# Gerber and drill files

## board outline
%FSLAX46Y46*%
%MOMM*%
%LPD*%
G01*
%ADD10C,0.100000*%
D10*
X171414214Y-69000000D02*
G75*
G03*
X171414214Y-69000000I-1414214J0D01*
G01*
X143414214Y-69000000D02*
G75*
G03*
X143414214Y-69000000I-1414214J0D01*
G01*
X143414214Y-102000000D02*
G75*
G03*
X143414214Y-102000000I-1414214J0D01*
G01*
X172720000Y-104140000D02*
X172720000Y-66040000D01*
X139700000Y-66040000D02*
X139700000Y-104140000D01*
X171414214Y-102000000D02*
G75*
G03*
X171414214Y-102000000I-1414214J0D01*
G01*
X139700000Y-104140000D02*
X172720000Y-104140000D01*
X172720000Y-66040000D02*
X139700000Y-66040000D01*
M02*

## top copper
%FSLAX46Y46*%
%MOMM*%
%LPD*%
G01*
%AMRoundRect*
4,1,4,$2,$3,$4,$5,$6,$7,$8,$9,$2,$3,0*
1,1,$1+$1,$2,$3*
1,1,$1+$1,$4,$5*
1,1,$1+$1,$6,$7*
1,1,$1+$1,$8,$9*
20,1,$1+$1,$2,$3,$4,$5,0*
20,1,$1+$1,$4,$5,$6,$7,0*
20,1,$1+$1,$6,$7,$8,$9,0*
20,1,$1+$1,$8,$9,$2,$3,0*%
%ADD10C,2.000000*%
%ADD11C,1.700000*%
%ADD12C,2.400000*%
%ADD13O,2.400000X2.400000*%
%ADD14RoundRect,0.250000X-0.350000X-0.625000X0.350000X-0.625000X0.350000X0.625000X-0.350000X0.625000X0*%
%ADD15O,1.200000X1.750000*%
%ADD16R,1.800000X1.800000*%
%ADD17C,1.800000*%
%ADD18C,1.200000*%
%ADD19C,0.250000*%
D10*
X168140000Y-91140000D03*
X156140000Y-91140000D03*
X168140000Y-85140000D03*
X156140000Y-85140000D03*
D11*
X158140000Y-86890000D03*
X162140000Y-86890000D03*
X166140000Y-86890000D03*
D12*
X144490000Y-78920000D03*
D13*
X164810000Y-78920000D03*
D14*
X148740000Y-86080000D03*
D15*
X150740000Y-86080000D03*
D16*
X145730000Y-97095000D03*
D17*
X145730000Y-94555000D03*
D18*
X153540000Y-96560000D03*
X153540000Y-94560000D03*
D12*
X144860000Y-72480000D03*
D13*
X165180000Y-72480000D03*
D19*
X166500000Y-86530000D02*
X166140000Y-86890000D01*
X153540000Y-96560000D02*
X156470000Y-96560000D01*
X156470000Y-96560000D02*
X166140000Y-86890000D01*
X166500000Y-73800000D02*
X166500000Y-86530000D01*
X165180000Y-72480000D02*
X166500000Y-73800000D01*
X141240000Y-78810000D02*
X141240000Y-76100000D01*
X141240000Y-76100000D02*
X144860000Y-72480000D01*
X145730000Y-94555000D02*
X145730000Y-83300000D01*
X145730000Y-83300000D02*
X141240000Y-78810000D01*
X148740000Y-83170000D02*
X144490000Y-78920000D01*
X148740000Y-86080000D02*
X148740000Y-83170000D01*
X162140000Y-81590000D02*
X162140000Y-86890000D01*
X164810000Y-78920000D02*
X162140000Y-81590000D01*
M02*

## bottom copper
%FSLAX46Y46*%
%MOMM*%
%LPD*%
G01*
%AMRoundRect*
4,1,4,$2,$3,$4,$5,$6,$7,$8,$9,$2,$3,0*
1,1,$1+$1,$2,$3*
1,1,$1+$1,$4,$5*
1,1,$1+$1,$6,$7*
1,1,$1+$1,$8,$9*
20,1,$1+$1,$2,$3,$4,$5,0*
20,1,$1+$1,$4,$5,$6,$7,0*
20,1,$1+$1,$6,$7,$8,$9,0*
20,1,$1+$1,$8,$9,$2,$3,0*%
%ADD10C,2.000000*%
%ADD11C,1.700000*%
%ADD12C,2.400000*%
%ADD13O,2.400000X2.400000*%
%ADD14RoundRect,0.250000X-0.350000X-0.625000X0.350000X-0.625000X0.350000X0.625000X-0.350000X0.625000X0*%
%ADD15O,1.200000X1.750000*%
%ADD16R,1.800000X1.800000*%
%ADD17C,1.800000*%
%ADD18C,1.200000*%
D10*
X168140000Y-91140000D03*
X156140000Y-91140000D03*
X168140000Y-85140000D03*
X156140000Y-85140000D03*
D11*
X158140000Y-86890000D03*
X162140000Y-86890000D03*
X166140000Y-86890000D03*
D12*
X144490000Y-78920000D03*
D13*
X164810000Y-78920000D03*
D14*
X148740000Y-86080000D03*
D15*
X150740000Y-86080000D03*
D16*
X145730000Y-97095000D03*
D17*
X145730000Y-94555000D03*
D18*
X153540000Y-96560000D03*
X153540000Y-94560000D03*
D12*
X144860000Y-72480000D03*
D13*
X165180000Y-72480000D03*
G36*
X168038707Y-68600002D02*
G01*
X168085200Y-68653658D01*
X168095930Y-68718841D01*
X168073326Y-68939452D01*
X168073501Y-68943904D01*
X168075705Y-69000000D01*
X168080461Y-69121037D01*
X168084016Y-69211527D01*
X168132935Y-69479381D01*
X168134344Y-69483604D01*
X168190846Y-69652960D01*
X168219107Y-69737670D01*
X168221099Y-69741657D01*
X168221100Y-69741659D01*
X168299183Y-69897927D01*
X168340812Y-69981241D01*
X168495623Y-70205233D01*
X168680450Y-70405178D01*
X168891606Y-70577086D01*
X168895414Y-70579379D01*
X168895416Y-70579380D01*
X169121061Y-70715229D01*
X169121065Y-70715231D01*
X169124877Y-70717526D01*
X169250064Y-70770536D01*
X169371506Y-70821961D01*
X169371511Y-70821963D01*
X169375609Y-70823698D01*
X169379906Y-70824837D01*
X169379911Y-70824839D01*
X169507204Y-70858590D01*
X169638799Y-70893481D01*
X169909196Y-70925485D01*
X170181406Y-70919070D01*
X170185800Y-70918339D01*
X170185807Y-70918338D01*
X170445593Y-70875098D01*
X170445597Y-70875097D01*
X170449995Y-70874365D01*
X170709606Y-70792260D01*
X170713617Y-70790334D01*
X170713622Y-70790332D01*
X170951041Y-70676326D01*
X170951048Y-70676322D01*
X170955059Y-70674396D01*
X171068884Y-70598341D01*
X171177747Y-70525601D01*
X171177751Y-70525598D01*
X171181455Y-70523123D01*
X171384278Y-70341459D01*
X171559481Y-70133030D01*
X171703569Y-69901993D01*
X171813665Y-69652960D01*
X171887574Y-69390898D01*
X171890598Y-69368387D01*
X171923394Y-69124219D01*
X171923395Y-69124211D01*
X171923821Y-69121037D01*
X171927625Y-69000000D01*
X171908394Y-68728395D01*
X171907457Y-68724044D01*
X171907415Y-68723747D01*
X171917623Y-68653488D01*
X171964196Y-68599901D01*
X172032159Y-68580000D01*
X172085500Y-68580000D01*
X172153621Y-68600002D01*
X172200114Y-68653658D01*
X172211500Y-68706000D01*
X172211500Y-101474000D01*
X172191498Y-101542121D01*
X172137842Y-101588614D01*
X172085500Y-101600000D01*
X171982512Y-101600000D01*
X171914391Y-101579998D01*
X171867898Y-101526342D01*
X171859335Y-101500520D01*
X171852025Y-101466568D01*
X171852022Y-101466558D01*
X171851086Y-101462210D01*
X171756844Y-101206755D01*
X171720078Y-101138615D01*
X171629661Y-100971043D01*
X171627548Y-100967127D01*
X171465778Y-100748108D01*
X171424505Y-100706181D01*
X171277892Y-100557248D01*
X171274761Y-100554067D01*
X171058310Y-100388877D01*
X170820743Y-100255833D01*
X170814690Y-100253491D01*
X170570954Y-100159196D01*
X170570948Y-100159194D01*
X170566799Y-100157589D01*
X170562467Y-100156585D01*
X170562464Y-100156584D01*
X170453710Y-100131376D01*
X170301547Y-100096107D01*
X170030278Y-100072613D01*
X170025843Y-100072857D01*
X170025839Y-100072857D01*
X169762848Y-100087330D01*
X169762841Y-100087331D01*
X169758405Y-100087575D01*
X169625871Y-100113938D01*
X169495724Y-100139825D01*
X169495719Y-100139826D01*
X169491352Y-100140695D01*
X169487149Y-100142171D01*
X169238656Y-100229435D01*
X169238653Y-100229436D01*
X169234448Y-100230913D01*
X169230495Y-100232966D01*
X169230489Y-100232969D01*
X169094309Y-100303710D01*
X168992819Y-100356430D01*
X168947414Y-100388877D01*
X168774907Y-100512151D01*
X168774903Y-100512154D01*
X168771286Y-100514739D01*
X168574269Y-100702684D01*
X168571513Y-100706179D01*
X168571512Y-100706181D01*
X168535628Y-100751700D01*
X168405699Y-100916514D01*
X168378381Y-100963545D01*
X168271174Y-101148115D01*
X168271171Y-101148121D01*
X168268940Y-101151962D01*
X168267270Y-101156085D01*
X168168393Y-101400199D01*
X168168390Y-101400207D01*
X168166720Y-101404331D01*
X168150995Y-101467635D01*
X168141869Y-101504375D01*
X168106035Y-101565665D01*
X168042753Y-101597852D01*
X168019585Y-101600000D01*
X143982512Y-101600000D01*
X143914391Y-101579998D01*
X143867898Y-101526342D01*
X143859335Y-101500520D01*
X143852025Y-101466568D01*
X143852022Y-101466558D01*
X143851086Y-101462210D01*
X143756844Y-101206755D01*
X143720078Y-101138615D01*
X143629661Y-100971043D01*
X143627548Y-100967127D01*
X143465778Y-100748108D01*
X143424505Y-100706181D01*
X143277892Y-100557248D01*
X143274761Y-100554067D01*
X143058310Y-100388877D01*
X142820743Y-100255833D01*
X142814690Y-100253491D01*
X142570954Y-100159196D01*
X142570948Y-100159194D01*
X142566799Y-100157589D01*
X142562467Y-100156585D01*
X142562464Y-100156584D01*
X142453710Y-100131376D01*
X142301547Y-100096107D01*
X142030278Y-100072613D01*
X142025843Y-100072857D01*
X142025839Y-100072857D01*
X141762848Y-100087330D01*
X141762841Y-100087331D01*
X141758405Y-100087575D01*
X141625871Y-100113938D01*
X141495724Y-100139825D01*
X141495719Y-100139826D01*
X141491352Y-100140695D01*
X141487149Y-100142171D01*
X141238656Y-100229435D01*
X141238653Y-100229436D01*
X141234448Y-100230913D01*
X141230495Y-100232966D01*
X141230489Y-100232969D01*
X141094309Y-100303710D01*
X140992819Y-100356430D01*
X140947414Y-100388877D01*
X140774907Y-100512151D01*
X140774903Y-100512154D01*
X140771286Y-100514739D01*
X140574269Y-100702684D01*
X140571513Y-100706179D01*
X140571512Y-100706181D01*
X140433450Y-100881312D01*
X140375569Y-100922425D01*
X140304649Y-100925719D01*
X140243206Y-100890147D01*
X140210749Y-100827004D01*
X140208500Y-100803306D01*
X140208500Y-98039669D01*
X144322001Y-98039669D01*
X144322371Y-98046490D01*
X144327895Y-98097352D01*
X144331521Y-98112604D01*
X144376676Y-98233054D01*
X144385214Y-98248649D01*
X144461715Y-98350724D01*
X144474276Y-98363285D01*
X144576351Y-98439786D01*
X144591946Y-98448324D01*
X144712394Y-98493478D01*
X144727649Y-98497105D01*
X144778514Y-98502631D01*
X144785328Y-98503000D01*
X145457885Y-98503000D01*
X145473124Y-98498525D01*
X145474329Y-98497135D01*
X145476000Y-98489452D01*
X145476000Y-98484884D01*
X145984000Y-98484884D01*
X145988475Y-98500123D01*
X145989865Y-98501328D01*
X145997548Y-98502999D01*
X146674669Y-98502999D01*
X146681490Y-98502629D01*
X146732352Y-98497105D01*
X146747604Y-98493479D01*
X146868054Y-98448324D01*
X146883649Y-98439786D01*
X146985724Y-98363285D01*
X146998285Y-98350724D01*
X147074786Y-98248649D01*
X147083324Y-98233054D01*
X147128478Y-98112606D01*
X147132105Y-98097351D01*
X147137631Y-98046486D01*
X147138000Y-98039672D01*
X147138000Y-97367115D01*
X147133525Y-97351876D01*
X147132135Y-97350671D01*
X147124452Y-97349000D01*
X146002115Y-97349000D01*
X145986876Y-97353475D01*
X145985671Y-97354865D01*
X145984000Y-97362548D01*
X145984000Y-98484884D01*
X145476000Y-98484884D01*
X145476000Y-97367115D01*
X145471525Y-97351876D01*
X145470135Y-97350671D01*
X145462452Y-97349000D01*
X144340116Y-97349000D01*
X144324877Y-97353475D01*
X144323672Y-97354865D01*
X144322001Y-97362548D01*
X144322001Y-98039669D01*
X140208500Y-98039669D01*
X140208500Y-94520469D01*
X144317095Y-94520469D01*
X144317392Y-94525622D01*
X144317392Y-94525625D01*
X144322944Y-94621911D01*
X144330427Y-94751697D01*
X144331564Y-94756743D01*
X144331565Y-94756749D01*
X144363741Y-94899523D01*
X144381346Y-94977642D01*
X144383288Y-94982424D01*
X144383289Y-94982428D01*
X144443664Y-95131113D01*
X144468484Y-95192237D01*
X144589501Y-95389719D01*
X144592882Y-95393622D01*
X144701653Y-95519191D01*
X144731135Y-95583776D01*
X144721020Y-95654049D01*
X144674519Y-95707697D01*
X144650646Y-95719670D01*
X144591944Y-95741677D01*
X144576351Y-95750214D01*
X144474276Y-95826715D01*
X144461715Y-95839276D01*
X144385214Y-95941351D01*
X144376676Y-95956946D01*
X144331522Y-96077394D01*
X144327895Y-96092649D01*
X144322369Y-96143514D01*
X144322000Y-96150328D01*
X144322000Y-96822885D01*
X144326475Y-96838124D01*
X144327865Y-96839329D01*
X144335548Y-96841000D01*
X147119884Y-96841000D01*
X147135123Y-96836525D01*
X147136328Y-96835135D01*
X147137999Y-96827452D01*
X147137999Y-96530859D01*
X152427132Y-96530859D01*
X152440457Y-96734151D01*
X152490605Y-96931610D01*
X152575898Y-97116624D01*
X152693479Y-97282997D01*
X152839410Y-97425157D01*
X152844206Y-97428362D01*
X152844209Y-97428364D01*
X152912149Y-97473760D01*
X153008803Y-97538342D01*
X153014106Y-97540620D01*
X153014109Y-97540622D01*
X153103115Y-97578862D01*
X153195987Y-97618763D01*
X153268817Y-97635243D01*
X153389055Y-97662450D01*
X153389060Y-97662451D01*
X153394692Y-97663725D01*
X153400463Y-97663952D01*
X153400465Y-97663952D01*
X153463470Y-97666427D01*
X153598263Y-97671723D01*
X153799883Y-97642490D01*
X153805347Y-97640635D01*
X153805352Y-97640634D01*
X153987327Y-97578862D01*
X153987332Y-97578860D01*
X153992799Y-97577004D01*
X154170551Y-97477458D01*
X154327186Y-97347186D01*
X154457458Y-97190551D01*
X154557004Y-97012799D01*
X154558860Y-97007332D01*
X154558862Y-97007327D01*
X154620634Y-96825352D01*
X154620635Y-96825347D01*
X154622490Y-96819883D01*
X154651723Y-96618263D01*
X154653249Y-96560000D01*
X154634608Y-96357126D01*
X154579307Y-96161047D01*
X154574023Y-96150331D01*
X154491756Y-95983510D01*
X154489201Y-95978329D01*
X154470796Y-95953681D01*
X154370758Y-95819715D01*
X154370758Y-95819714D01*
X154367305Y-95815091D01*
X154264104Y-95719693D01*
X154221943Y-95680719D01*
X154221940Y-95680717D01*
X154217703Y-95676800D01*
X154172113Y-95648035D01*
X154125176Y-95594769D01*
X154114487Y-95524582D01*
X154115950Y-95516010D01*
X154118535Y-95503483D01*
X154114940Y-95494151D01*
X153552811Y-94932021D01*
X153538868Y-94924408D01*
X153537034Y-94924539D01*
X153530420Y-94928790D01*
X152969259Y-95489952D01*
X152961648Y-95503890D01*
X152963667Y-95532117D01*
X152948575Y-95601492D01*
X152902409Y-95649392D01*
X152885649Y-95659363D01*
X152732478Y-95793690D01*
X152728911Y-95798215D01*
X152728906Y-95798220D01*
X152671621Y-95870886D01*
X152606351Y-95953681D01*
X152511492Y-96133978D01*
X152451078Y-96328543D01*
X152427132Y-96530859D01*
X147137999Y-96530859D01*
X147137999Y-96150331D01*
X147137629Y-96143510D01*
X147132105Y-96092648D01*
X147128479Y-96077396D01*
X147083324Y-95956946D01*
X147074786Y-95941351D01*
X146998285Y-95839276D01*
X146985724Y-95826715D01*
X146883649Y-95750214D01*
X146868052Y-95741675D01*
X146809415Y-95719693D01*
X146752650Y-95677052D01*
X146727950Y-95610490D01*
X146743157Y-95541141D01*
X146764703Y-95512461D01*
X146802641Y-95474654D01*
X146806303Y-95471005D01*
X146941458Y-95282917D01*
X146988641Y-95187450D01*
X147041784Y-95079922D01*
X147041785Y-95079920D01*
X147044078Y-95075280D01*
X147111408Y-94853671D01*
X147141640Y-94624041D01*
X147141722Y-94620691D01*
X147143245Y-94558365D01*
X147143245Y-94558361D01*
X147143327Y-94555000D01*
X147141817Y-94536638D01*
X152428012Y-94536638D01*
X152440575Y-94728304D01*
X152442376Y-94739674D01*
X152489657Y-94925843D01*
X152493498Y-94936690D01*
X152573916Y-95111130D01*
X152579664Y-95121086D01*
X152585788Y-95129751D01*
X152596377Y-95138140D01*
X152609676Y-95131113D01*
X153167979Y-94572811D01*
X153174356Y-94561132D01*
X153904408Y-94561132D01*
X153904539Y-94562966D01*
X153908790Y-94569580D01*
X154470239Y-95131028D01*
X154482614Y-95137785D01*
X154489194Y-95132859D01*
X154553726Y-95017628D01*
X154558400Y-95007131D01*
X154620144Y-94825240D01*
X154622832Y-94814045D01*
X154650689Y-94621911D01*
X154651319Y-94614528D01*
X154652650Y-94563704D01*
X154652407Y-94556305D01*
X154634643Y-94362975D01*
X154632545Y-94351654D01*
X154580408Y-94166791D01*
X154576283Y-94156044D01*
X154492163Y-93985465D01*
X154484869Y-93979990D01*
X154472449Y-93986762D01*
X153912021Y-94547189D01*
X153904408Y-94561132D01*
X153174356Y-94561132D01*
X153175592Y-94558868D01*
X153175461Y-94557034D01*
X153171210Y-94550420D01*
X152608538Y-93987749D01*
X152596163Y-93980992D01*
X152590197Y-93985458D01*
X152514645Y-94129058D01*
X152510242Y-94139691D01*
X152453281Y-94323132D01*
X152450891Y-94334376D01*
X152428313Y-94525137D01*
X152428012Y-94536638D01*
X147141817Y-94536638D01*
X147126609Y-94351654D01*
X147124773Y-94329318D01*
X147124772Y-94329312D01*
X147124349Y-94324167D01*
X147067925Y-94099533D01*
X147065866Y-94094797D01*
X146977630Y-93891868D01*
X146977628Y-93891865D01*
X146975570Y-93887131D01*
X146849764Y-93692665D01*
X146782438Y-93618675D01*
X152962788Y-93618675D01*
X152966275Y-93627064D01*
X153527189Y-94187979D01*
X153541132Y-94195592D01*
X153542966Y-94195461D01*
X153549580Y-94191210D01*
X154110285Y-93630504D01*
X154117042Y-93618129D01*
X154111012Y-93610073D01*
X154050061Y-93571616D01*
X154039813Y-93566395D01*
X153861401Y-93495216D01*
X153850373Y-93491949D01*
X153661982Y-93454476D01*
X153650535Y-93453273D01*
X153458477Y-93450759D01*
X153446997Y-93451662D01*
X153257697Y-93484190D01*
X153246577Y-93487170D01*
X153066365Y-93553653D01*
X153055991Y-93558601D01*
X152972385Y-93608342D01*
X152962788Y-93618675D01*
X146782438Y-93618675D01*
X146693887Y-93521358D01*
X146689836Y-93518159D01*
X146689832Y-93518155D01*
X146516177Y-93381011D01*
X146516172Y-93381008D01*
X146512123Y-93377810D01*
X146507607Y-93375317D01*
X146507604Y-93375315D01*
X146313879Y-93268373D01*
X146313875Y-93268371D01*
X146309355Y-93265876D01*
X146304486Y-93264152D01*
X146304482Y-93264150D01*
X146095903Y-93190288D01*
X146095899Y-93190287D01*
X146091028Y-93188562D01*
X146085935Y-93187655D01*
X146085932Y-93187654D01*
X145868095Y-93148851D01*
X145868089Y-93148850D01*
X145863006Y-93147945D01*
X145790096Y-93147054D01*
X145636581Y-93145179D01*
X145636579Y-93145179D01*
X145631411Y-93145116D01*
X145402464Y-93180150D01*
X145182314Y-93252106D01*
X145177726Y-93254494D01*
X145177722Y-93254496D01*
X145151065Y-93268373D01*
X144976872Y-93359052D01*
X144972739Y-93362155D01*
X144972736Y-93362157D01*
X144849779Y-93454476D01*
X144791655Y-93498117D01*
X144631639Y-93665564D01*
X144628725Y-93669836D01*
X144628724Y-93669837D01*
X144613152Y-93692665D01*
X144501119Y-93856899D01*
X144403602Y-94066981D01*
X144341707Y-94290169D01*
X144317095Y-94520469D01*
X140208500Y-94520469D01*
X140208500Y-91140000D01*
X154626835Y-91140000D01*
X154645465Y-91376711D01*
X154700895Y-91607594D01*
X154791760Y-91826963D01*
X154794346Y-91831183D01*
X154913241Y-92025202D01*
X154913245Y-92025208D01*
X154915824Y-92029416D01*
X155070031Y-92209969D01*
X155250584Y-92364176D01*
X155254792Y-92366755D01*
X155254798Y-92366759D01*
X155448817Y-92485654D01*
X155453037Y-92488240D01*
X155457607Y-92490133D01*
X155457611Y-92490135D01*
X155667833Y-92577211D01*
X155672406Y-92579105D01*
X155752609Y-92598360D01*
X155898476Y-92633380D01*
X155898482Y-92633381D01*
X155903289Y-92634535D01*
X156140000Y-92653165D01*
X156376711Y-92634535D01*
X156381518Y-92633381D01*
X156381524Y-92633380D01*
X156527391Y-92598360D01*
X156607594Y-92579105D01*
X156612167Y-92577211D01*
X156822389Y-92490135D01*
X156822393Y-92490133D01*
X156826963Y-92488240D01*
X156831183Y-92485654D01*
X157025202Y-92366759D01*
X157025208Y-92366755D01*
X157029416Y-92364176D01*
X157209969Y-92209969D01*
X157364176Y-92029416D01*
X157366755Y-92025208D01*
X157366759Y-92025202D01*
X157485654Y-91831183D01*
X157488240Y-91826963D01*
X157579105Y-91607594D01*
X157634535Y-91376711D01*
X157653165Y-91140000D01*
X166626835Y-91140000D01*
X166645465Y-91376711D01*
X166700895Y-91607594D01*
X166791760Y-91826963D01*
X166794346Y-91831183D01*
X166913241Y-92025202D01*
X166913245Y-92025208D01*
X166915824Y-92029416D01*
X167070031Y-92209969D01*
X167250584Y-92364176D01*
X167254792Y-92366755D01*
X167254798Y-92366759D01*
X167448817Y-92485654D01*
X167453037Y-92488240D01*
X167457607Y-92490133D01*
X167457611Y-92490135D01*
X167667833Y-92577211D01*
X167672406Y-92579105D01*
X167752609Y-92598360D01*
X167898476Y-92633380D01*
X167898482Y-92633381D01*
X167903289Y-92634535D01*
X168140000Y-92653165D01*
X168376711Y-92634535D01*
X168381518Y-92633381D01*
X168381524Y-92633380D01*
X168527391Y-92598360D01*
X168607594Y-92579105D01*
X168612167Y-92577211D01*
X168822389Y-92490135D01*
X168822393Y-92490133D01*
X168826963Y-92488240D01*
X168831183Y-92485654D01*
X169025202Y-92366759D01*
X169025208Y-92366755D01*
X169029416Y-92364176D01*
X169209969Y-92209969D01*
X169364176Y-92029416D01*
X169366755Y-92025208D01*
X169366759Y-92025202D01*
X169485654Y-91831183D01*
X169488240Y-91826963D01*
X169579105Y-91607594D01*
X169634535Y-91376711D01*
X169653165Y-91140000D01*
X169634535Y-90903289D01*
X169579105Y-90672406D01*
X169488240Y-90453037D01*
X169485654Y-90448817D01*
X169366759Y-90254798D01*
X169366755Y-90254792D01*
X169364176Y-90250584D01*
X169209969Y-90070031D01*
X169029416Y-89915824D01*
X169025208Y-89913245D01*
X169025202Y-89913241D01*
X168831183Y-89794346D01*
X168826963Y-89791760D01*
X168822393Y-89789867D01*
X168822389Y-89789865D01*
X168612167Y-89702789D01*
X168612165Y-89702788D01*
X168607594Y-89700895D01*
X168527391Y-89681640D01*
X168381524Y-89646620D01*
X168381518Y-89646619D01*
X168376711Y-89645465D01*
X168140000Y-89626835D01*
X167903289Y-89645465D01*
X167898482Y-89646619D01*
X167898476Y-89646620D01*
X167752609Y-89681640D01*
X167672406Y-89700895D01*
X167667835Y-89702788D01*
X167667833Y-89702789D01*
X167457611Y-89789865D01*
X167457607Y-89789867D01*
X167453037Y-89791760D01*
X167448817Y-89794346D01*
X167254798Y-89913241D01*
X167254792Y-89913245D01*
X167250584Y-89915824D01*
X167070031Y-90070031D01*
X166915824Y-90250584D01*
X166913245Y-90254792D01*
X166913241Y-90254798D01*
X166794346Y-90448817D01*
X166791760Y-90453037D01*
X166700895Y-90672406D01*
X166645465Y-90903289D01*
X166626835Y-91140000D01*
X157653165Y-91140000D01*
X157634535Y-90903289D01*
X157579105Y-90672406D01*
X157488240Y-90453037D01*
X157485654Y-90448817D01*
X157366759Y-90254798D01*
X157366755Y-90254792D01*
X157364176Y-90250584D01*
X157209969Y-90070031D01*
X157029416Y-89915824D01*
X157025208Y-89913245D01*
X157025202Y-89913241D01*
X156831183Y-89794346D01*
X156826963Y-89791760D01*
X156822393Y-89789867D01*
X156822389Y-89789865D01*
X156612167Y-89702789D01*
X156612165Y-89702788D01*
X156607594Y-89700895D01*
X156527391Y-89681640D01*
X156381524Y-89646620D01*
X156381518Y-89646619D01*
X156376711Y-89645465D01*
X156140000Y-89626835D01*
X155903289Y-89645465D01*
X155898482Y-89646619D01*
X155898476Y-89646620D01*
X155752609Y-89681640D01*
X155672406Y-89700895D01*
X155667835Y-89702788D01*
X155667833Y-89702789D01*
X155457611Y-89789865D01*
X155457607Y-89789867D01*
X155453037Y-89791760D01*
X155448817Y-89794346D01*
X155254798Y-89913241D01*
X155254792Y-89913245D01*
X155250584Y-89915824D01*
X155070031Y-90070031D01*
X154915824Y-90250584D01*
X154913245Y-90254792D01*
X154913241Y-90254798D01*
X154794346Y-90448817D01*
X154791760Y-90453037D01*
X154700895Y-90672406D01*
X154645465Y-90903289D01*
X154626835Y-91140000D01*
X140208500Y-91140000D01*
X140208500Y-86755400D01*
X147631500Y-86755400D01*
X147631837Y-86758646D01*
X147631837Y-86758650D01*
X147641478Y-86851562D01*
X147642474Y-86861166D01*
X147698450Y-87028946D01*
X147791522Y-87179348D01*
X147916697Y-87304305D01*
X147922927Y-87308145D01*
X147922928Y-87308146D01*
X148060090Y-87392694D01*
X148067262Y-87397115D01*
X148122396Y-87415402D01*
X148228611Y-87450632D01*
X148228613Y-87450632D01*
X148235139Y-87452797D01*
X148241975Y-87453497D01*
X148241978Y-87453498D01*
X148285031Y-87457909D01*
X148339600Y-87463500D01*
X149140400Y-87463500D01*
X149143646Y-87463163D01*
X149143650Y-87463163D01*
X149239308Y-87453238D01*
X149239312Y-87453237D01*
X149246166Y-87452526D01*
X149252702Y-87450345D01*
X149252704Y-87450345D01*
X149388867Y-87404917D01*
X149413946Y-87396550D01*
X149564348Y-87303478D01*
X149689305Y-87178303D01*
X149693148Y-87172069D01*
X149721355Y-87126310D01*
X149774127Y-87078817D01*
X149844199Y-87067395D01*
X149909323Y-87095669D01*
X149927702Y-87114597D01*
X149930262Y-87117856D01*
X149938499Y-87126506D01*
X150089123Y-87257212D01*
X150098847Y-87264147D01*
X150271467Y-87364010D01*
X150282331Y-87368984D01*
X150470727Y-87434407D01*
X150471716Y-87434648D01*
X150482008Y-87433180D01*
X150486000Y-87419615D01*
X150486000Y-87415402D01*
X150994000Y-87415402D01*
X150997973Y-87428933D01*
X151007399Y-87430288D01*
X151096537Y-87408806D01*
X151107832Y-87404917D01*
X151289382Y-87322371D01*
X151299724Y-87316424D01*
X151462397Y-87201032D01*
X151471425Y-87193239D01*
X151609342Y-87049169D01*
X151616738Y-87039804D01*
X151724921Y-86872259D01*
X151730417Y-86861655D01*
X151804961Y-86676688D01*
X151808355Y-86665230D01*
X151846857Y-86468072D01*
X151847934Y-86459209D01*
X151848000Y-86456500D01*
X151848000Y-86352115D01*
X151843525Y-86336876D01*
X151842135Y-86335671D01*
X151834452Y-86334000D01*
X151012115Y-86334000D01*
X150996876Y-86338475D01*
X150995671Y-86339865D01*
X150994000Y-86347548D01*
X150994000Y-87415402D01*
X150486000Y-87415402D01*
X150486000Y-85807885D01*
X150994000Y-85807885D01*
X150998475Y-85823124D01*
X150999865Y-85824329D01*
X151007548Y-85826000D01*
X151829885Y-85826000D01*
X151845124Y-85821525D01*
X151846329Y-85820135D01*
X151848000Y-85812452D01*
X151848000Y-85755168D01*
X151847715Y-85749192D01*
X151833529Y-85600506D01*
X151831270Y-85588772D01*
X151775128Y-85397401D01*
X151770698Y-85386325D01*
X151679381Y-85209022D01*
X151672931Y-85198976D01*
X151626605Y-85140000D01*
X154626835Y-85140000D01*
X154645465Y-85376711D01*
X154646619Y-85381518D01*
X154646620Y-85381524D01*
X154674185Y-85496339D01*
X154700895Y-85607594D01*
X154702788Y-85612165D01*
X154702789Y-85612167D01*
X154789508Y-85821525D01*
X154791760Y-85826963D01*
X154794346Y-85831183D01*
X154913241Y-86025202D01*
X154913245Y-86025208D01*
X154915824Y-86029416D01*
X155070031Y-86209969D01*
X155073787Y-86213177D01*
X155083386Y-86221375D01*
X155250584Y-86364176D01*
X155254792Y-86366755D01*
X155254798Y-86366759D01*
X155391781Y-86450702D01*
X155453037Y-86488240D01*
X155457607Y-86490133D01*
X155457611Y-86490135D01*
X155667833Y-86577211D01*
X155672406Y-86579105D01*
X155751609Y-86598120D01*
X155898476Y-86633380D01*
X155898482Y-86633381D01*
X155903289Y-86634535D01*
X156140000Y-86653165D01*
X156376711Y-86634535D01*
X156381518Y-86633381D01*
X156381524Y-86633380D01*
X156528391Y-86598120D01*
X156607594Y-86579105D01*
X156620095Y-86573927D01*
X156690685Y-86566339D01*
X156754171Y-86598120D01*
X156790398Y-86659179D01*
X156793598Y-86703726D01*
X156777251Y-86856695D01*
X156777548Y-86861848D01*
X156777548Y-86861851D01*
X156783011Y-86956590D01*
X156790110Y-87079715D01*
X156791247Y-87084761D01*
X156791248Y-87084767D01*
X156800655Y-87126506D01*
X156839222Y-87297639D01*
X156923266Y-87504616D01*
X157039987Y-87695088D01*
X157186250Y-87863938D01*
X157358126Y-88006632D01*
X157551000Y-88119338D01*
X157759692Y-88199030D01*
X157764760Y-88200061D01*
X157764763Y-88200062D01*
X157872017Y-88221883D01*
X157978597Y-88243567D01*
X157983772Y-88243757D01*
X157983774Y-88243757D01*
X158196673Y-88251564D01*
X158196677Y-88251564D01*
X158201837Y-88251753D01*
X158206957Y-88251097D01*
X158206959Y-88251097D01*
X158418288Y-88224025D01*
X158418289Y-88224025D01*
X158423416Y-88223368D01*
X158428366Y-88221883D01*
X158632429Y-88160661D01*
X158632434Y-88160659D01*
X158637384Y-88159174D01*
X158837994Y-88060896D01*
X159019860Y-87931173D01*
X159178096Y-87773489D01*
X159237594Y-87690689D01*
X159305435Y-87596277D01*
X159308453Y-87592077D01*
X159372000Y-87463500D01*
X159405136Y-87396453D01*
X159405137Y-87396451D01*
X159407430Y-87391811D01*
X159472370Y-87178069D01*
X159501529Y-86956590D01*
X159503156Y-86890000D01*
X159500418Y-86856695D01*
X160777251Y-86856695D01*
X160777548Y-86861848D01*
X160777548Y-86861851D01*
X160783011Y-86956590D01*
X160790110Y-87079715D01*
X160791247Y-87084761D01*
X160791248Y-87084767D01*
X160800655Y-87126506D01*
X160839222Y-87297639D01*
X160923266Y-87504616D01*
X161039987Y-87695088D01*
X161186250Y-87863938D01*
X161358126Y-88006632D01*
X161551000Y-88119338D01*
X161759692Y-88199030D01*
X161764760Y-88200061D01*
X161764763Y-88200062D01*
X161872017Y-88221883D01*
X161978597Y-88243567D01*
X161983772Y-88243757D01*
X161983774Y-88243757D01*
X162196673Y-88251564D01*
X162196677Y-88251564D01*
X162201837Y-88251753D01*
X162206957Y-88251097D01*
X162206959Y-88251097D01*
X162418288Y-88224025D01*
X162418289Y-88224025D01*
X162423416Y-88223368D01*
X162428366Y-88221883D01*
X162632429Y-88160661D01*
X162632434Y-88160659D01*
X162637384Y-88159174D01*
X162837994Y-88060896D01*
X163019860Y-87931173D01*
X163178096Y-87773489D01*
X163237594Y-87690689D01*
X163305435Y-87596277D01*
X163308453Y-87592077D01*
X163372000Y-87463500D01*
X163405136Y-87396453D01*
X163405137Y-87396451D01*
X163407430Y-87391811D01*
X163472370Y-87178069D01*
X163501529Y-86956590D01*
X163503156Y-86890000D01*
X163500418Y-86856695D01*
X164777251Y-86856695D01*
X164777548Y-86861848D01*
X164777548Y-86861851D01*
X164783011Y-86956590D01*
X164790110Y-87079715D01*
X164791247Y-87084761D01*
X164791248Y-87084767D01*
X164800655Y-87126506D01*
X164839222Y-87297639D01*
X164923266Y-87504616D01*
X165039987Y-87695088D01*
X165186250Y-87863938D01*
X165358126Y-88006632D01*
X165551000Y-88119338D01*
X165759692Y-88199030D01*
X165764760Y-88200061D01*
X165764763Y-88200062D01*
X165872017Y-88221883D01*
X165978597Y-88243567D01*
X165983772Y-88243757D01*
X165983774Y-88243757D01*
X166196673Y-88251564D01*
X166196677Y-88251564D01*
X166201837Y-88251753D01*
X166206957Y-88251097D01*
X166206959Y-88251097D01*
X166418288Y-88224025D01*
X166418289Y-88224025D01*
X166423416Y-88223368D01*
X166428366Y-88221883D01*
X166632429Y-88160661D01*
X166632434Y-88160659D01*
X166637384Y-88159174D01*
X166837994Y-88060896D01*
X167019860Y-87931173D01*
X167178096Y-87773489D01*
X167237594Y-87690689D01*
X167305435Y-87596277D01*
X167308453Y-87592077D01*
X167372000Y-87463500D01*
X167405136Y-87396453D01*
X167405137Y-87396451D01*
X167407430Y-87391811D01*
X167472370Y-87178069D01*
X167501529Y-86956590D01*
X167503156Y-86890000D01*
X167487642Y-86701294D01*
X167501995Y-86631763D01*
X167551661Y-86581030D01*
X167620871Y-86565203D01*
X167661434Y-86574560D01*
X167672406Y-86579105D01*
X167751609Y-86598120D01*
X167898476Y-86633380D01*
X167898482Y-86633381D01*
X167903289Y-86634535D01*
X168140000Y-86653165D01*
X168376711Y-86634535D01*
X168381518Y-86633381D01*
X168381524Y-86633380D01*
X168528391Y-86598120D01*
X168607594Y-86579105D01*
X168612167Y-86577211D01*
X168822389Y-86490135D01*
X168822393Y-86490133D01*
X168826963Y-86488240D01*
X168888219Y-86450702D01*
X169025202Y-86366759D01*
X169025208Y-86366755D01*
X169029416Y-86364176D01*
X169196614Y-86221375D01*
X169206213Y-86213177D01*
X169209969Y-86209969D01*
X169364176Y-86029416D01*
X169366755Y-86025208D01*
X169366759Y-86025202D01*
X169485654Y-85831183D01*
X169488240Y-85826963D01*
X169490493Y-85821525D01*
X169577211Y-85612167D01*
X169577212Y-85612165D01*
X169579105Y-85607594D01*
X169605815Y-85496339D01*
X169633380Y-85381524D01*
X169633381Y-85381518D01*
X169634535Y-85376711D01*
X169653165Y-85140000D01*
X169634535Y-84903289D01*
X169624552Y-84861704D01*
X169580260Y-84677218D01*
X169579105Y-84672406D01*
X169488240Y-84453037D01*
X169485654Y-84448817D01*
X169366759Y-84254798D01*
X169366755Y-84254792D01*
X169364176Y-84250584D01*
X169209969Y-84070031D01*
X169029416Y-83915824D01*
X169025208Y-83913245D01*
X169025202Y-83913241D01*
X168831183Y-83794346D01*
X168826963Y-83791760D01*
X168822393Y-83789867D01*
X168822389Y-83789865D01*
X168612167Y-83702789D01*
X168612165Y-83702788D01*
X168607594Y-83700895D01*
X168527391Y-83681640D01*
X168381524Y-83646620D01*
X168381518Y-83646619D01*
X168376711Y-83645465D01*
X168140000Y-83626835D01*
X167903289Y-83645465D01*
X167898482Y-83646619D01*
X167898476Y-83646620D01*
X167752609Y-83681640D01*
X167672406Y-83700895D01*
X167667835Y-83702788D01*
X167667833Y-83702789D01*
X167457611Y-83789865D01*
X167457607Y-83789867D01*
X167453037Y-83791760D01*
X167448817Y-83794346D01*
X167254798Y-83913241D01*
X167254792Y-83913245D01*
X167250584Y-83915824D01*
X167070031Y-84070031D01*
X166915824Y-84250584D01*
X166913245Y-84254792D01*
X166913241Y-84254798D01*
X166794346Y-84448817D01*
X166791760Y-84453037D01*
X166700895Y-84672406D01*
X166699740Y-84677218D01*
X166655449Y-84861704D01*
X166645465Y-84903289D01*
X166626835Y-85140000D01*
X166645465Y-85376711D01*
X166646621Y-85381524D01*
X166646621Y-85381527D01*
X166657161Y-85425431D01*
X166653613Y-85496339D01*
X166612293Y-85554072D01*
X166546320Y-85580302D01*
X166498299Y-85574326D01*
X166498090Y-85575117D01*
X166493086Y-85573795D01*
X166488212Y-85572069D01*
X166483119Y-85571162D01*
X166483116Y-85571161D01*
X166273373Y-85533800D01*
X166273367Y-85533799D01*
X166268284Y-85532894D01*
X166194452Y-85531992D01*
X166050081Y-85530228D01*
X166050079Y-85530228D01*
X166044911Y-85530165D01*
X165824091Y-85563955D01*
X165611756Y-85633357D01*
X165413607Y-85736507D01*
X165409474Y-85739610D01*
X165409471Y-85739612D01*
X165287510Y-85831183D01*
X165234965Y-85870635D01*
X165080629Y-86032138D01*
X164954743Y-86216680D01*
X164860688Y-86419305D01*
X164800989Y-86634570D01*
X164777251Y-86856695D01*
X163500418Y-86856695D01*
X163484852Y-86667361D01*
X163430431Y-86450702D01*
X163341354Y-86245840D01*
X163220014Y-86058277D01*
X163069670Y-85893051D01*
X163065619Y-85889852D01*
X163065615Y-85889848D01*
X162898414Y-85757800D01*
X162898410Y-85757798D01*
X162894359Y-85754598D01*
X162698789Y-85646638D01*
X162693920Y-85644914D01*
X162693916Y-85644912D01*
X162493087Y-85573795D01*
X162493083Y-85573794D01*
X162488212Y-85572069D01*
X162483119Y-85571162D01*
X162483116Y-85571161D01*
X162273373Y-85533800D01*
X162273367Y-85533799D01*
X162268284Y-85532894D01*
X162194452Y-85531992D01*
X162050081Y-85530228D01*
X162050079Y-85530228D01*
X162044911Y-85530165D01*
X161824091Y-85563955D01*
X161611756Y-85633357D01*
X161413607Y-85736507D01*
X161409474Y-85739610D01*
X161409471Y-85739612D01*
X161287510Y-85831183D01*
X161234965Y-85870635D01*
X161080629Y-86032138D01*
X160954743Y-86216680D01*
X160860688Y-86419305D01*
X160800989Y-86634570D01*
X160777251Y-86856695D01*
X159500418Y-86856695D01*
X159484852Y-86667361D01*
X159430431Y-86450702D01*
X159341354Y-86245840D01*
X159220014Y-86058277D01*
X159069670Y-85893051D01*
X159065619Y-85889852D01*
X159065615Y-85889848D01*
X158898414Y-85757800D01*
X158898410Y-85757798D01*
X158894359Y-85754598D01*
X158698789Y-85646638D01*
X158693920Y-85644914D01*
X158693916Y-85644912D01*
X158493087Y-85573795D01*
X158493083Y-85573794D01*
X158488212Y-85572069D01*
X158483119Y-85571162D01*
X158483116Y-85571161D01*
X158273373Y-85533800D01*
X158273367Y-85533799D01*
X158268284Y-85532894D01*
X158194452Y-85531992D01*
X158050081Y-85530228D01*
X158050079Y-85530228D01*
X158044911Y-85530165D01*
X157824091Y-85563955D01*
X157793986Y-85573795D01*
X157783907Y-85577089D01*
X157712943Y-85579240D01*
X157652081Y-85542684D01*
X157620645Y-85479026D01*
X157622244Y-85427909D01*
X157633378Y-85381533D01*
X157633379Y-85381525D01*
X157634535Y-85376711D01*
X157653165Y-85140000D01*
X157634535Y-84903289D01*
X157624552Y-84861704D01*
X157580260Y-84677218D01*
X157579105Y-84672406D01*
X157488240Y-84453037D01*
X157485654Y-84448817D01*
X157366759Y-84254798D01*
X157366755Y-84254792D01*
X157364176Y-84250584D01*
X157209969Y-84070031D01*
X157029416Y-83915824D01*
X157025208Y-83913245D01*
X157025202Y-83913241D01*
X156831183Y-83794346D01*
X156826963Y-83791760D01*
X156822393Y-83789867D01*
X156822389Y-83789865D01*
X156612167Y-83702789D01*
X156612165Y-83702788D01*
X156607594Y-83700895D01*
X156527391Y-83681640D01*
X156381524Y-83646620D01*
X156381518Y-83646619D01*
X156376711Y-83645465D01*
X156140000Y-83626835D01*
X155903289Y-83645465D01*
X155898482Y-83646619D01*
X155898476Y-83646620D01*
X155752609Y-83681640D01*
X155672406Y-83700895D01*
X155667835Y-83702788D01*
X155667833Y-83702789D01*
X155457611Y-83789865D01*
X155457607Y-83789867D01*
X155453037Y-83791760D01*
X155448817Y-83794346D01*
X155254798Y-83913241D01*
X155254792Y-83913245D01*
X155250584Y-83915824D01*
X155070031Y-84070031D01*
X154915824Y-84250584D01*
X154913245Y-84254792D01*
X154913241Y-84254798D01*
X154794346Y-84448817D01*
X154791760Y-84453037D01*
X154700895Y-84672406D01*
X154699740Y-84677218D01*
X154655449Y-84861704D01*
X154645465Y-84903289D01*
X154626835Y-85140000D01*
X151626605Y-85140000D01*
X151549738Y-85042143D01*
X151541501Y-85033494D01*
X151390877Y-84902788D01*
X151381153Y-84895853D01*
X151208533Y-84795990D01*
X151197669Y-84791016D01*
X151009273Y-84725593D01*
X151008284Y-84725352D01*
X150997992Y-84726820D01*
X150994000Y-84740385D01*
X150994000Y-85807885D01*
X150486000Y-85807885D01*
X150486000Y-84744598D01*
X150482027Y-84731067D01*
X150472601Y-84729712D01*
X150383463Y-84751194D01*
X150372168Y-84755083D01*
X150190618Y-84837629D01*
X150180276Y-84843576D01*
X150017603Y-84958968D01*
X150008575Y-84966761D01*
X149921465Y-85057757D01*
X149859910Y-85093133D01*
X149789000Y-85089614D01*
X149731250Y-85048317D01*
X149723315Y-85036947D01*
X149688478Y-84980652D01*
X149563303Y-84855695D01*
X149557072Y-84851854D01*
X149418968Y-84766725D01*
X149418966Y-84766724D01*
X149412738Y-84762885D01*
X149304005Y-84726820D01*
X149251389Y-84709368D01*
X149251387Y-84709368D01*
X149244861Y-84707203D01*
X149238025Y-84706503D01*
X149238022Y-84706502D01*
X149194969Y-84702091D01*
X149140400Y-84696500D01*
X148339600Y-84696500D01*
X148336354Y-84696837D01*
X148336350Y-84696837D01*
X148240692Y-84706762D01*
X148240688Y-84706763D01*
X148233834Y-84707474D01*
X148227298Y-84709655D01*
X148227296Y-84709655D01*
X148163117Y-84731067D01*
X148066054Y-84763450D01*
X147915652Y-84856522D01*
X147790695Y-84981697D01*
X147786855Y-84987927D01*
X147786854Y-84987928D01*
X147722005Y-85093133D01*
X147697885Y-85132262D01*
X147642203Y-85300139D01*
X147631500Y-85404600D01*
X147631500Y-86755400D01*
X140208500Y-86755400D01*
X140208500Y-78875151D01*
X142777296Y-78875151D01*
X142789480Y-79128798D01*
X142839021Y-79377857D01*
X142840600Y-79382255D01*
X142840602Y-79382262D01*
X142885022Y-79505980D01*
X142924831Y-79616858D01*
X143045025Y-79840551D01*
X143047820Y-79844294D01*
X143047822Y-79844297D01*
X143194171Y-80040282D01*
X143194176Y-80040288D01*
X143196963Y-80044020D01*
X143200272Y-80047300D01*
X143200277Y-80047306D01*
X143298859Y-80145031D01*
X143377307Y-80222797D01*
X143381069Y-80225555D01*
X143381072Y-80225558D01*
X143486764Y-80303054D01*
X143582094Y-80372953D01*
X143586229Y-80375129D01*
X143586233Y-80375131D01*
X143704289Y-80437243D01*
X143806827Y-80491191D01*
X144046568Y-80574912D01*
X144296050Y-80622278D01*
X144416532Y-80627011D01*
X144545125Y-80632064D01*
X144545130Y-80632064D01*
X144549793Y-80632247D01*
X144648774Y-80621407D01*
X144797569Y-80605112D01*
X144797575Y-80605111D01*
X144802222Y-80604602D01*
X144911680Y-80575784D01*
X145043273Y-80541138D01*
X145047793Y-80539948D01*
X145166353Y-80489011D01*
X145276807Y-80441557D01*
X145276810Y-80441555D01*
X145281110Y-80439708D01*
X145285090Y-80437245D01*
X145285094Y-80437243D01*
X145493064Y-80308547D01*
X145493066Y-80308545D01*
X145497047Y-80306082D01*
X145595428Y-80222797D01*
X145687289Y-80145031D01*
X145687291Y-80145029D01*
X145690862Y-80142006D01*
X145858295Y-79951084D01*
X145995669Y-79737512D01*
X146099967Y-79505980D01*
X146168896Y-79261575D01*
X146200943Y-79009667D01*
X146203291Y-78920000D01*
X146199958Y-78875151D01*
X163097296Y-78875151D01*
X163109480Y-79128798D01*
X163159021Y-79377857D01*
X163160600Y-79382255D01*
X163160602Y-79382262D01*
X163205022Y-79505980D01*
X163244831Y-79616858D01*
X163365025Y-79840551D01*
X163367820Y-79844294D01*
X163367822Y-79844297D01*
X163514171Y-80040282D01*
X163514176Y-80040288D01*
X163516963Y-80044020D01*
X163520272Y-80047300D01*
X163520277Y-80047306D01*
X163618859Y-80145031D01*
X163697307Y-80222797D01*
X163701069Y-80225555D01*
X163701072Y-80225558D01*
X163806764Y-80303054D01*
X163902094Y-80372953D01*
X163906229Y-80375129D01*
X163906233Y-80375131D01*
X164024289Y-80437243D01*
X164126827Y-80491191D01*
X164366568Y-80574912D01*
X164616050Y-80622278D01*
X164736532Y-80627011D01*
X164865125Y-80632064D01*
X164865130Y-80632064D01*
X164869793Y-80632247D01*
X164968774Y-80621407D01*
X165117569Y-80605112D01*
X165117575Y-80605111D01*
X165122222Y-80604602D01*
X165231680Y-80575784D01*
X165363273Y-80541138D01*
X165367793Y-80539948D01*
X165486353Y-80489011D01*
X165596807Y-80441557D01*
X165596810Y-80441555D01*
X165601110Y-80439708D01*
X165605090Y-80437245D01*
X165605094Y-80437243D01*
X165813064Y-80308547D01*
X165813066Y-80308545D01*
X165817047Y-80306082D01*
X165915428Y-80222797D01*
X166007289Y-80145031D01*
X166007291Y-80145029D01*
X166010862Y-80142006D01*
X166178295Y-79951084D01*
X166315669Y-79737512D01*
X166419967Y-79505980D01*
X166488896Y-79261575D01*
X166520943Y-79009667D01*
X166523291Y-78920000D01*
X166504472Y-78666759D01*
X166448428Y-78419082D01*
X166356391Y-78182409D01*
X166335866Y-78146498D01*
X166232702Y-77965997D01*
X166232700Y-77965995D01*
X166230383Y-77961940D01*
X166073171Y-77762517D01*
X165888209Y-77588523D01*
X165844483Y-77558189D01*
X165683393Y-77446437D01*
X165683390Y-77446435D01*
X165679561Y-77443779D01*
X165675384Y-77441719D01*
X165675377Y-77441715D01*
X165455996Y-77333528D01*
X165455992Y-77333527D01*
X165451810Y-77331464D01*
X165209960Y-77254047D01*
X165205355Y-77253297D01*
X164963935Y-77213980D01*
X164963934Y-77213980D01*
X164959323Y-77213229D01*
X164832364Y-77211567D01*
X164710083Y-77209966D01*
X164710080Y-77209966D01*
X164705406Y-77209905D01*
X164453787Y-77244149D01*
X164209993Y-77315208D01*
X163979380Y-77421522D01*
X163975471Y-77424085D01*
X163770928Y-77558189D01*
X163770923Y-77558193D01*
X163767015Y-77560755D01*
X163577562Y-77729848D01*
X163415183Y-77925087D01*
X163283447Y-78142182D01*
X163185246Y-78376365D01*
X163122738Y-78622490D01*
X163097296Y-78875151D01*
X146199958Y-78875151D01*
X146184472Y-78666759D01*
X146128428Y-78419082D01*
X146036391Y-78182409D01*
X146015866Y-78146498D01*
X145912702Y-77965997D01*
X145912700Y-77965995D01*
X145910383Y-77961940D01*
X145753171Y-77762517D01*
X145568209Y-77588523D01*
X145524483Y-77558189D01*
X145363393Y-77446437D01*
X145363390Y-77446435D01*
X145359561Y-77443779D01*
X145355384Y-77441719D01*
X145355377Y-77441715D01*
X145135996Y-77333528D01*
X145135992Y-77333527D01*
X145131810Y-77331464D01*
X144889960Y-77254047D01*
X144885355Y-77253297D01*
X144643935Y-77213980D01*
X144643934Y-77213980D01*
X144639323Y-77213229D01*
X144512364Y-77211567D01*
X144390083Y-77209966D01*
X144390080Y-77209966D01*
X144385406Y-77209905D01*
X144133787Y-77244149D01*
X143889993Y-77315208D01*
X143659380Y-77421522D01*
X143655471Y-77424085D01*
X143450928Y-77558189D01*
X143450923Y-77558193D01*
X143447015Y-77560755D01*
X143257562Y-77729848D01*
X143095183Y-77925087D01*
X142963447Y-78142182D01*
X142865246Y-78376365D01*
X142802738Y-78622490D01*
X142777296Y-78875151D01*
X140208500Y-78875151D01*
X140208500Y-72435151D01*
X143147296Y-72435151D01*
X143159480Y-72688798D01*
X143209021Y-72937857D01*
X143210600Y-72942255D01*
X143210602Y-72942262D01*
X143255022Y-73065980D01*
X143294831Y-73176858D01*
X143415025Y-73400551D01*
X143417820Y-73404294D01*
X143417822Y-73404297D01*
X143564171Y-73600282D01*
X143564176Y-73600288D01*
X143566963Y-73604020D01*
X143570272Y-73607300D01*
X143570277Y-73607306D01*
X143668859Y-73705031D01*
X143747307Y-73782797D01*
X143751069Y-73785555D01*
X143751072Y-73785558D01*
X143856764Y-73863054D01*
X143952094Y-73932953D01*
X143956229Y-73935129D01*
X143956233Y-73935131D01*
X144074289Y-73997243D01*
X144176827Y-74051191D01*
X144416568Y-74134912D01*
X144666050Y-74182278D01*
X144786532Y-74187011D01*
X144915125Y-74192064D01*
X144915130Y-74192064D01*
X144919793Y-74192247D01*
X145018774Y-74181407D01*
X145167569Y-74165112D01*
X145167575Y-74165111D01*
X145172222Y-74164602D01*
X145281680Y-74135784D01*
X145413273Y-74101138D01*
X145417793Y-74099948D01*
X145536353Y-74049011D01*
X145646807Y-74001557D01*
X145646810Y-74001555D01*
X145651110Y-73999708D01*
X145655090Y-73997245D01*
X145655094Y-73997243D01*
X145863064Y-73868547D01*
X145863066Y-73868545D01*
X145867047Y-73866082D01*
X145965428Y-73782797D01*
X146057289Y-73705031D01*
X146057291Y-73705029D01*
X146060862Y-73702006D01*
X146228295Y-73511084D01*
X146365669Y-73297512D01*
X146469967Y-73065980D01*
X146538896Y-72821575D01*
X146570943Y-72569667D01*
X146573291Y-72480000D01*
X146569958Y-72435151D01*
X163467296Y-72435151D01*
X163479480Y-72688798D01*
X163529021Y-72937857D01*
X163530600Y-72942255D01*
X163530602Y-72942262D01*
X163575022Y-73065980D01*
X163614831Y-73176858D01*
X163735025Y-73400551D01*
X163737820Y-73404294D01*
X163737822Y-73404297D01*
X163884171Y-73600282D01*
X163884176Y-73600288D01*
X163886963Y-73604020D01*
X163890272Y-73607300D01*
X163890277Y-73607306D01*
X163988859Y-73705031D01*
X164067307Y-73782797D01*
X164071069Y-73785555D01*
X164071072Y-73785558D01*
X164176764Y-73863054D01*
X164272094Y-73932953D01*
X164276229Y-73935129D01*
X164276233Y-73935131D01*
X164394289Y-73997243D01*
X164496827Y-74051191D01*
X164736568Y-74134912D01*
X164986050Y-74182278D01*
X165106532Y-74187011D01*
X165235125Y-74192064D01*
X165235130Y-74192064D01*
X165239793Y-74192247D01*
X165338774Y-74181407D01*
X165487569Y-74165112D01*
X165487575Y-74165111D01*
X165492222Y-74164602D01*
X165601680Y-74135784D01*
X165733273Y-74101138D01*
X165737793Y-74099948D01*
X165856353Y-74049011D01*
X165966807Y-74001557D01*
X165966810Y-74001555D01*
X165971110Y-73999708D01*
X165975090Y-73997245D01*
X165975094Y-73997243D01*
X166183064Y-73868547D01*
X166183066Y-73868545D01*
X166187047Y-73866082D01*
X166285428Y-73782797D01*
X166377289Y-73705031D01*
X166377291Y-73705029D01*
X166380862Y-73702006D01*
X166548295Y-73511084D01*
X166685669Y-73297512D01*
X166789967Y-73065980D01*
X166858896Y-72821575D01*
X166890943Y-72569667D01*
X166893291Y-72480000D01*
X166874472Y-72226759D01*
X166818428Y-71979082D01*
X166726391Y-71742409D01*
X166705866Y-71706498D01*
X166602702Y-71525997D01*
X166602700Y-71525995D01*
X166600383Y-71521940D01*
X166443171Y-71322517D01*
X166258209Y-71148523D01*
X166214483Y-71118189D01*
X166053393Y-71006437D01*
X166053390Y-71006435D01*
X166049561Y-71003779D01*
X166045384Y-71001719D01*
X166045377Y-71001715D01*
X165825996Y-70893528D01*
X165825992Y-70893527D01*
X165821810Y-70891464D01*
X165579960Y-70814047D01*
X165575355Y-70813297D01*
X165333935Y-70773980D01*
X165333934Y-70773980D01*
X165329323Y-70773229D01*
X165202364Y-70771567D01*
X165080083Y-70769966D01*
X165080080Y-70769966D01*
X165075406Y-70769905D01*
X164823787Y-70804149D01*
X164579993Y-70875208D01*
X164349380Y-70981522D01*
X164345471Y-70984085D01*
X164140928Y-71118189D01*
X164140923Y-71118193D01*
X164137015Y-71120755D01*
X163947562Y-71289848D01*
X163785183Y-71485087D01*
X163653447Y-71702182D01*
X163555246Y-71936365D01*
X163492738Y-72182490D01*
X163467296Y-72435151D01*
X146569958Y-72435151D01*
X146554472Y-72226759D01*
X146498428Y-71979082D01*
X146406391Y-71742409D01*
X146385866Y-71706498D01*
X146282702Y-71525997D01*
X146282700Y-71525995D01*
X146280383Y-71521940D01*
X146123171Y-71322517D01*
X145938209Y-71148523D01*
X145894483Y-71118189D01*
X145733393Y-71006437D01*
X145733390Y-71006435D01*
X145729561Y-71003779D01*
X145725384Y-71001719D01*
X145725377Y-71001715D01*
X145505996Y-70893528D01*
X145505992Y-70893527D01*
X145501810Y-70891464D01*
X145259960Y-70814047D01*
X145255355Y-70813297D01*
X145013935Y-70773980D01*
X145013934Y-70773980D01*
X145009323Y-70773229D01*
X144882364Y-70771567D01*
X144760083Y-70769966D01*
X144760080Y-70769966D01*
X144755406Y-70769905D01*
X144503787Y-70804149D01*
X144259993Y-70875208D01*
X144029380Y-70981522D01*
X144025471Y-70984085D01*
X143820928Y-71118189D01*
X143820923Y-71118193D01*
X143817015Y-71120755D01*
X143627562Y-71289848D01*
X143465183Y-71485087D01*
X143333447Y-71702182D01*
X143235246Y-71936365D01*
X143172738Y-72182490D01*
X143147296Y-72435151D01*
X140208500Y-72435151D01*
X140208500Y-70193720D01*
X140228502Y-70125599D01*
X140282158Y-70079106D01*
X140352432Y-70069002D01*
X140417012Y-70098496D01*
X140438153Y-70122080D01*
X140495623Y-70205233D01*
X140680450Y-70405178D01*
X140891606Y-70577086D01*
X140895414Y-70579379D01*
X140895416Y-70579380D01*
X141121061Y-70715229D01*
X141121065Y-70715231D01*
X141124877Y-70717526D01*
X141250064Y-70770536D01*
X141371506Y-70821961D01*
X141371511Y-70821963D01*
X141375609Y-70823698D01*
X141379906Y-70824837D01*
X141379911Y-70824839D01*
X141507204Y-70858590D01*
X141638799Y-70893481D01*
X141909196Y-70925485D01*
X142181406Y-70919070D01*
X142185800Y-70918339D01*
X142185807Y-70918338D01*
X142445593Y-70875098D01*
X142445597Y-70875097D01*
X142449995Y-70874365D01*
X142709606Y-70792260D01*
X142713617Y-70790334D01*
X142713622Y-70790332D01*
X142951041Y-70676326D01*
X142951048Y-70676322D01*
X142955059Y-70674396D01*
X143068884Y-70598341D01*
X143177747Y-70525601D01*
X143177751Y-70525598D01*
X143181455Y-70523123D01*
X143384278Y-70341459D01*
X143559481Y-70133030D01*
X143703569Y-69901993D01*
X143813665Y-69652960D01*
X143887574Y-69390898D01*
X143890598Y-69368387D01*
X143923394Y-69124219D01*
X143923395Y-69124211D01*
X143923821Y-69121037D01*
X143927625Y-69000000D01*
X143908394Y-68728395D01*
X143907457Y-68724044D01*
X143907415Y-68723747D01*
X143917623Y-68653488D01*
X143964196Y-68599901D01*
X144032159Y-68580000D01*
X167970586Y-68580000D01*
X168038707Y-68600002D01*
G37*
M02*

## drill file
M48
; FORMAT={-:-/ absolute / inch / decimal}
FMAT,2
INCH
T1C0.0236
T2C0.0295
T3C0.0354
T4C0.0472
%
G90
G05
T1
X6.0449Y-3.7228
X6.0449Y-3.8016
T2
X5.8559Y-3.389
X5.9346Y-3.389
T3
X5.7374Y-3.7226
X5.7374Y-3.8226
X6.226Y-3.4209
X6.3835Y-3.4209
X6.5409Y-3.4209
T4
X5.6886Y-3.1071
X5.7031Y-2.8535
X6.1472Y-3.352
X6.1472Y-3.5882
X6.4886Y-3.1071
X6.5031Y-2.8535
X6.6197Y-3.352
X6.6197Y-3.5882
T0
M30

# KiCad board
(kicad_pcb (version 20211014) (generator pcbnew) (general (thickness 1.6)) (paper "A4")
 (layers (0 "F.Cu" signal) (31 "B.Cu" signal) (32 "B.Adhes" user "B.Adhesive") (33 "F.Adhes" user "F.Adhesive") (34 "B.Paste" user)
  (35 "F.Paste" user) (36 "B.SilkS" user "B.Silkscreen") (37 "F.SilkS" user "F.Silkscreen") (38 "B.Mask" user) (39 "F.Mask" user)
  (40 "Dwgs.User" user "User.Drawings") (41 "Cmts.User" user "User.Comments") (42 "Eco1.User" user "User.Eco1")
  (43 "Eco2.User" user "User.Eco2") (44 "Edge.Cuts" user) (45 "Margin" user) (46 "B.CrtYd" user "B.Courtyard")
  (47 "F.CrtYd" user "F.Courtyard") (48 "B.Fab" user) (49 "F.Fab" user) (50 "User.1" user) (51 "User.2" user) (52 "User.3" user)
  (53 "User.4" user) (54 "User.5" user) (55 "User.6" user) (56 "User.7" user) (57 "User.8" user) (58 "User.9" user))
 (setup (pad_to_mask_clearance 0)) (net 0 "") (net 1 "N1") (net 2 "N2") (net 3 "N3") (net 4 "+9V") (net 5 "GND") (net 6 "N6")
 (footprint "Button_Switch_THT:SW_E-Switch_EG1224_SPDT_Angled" (layer "F.Cu") (at 158.14 86.89)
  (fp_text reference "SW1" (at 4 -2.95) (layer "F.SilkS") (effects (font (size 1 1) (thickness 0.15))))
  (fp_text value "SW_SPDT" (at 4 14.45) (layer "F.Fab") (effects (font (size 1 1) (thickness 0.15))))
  (pad "" thru_hole circle (at 10 4.25) (size 2 2) (drill 1.2) (layers *.Cu *.Mask))
  (pad "" thru_hole circle (at -2 4.25) (size 2 2) (drill 1.2) (layers *.Cu *.Mask))
  (pad "" thru_hole circle (at 10 -1.75) (size 2 2) (drill 1.2) (layers *.Cu *.Mask))
  (pad "" thru_hole circle (at -2 -1.75) (size 2 2) (drill 1.2) (layers *.Cu *.Mask))
  (pad "1" thru_hole circle (at 0 0) (size 1.7 1.7) (drill 0.9) (layers *.Cu *.Mask) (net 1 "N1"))
  (pad "2" thru_hole circle (at 4 0) (size 1.7 1.7) (drill 0.9) (layers *.Cu *.Mask) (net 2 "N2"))
  (pad "3" thru_hole circle (at 8 0) (size 1.7 1.7) (drill 0.9) (layers *.Cu *.Mask) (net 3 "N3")))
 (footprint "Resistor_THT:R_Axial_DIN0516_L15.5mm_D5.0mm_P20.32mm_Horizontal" (layer "F.Cu") (at 144.49 78.92)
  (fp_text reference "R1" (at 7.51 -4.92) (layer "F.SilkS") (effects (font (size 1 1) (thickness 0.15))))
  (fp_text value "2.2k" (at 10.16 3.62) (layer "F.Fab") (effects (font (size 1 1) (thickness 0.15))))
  (pad "1" thru_hole circle (at 0 0) (size 2.4 2.4) (drill 1.2) (layers *.Cu *.Mask) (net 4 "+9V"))
  (pad "2" thru_hole oval (at 20.32 0) (size 2.4 2.4) (drill 1.2) (layers *.Cu *.Mask) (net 2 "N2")))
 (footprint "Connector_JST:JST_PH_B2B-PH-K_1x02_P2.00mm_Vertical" (layer "F.Cu") (at 148.74 86.08)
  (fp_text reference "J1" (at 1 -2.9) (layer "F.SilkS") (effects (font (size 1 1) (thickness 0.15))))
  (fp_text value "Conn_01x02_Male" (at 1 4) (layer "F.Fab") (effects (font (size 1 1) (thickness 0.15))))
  (pad "1" thru_hole roundrect (at 0 0) (size 1.2 1.75) (drill 0.75) (layers *.Cu *.Mask) (roundrect_rratio 0.2083333333) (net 4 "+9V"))
  (pad "2" thru_hole oval (at 2 0) (size 1.2 1.75) (drill 0.75) (layers *.Cu *.Mask) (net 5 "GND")))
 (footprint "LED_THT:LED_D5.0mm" (layer "F.Cu") (at 145.73 97.095 90)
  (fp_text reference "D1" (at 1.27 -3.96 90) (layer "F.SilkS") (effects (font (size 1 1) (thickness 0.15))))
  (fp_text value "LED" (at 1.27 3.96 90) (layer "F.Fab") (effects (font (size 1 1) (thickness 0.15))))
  (pad "1" thru_hole rect (at 0 0 90) (size 1.8 1.8) (drill 0.9) (layers *.Cu *.Mask) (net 5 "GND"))
  (pad "2" thru_hole circle (at 2.54 0 90) (size 1.8 1.8) (drill 0.9) (layers *.Cu *.Mask) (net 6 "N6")))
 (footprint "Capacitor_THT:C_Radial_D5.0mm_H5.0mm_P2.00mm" (layer "F.Cu") (at 153.54 96.56 90)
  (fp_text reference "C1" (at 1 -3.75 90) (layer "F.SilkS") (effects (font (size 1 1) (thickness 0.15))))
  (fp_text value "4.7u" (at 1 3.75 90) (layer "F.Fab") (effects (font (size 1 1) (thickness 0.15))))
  (pad "1" thru_hole circle (at 0 0 90) (size 1.2 1.2) (drill 0.6) (layers *.Cu *.Mask) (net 3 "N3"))
  (pad "2" thru_hole circle (at 2 0 90) (size 1.2 1.2) (drill 0.6) (layers *.Cu *.Mask) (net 5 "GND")))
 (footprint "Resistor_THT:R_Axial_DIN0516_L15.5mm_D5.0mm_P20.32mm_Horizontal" (layer "F.Cu") (at 144.86 72.48)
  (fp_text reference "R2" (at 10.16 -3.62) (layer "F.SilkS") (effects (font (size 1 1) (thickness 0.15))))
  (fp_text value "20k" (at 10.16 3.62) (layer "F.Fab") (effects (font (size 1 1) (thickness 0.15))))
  (pad "1" thru_hole circle (at 0 0) (size 2.4 2.4) (drill 1.2) (layers *.Cu *.Mask) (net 6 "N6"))
  (pad "2" thru_hole oval (at 20.32 0) (size 2.4 2.4) (drill 1.2) (layers *.Cu *.Mask) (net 3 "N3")))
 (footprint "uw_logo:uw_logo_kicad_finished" (layer "F.Cu") (at 148 102)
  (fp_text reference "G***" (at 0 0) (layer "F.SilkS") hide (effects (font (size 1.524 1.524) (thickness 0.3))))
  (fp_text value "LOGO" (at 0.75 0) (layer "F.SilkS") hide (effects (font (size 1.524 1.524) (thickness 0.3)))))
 (gr_circle (center 170 69) (end 169 68) (layer "Edge.Cuts") (width 0.1) (fill none))
 (gr_circle (center 142 69) (end 141 68) (layer "Edge.Cuts") (width 0.1) (fill none))
 (gr_circle (center 142 102) (end 141 103) (layer "Edge.Cuts") (width 0.1) (fill none))
 (gr_line (start 172.72 104.14) (end 172.72 66.04) (layer "Edge.Cuts") (width 0.1))
 (gr_line (start 139.7 66.04) (end 139.7 104.14) (layer "Edge.Cuts") (width 0.1))
 (gr_circle (center 170 102) (end 171 103) (layer "Edge.Cuts") (width 0.1) (fill none))
 (gr_line (start 139.7 104.14) (end 172.72 104.14) (layer "Edge.Cuts") (width 0.1))
 (gr_line (start 172.72 66.04) (end 139.7 66.04) (layer "Edge.Cuts") (width 0.1))
 (segment (start 166.5 86.53) (end 166.14 86.89) (width 0.25) (layer "F.Cu") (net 3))
 (segment (start 153.54 96.56) (end 156.47 96.56) (width 0.25) (layer "F.Cu") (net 3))
 (segment (start 156.47 96.56) (end 166.14 86.89) (width 0.25) (layer "F.Cu") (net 3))
 (segment (start 166.5 73.8) (end 166.5 86.53) (width 0.25) (layer "F.Cu") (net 3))
 (segment (start 165.18 72.48) (end 166.5 73.8) (width 0.25) (layer "F.Cu") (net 3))
 (segment (start 141.24 78.81) (end 141.24 76.1) (width 0.25) (layer "F.Cu") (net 6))
 (segment (start 141.24 76.1) (end 144.86 72.48) (width 0.25) (layer "F.Cu") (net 6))
 (segment (start 145.73 94.555) (end 145.73 83.3) (width 0.25) (layer "F.Cu") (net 6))
 (segment (start 145.73 83.3) (end 141.24 78.81) (width 0.25) (layer "F.Cu") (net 6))
 (segment (start 148.74 83.17) (end 144.49 78.92) (width 0.25) (layer "F.Cu") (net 4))
 (segment (start 148.74 86.08) (end 148.74 83.17) (width 0.25) (layer "F.Cu") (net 4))
 (segment (start 162.14 81.59) (end 162.14 86.89) (width 0.25) (layer "F.Cu") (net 2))
 (segment (start 164.81 78.92) (end 162.14 81.59) (width 0.25) (layer "F.Cu") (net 2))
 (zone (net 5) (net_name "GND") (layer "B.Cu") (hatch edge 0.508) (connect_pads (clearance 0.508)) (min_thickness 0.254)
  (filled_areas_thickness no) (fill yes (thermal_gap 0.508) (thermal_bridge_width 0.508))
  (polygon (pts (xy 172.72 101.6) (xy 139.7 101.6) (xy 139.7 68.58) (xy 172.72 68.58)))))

